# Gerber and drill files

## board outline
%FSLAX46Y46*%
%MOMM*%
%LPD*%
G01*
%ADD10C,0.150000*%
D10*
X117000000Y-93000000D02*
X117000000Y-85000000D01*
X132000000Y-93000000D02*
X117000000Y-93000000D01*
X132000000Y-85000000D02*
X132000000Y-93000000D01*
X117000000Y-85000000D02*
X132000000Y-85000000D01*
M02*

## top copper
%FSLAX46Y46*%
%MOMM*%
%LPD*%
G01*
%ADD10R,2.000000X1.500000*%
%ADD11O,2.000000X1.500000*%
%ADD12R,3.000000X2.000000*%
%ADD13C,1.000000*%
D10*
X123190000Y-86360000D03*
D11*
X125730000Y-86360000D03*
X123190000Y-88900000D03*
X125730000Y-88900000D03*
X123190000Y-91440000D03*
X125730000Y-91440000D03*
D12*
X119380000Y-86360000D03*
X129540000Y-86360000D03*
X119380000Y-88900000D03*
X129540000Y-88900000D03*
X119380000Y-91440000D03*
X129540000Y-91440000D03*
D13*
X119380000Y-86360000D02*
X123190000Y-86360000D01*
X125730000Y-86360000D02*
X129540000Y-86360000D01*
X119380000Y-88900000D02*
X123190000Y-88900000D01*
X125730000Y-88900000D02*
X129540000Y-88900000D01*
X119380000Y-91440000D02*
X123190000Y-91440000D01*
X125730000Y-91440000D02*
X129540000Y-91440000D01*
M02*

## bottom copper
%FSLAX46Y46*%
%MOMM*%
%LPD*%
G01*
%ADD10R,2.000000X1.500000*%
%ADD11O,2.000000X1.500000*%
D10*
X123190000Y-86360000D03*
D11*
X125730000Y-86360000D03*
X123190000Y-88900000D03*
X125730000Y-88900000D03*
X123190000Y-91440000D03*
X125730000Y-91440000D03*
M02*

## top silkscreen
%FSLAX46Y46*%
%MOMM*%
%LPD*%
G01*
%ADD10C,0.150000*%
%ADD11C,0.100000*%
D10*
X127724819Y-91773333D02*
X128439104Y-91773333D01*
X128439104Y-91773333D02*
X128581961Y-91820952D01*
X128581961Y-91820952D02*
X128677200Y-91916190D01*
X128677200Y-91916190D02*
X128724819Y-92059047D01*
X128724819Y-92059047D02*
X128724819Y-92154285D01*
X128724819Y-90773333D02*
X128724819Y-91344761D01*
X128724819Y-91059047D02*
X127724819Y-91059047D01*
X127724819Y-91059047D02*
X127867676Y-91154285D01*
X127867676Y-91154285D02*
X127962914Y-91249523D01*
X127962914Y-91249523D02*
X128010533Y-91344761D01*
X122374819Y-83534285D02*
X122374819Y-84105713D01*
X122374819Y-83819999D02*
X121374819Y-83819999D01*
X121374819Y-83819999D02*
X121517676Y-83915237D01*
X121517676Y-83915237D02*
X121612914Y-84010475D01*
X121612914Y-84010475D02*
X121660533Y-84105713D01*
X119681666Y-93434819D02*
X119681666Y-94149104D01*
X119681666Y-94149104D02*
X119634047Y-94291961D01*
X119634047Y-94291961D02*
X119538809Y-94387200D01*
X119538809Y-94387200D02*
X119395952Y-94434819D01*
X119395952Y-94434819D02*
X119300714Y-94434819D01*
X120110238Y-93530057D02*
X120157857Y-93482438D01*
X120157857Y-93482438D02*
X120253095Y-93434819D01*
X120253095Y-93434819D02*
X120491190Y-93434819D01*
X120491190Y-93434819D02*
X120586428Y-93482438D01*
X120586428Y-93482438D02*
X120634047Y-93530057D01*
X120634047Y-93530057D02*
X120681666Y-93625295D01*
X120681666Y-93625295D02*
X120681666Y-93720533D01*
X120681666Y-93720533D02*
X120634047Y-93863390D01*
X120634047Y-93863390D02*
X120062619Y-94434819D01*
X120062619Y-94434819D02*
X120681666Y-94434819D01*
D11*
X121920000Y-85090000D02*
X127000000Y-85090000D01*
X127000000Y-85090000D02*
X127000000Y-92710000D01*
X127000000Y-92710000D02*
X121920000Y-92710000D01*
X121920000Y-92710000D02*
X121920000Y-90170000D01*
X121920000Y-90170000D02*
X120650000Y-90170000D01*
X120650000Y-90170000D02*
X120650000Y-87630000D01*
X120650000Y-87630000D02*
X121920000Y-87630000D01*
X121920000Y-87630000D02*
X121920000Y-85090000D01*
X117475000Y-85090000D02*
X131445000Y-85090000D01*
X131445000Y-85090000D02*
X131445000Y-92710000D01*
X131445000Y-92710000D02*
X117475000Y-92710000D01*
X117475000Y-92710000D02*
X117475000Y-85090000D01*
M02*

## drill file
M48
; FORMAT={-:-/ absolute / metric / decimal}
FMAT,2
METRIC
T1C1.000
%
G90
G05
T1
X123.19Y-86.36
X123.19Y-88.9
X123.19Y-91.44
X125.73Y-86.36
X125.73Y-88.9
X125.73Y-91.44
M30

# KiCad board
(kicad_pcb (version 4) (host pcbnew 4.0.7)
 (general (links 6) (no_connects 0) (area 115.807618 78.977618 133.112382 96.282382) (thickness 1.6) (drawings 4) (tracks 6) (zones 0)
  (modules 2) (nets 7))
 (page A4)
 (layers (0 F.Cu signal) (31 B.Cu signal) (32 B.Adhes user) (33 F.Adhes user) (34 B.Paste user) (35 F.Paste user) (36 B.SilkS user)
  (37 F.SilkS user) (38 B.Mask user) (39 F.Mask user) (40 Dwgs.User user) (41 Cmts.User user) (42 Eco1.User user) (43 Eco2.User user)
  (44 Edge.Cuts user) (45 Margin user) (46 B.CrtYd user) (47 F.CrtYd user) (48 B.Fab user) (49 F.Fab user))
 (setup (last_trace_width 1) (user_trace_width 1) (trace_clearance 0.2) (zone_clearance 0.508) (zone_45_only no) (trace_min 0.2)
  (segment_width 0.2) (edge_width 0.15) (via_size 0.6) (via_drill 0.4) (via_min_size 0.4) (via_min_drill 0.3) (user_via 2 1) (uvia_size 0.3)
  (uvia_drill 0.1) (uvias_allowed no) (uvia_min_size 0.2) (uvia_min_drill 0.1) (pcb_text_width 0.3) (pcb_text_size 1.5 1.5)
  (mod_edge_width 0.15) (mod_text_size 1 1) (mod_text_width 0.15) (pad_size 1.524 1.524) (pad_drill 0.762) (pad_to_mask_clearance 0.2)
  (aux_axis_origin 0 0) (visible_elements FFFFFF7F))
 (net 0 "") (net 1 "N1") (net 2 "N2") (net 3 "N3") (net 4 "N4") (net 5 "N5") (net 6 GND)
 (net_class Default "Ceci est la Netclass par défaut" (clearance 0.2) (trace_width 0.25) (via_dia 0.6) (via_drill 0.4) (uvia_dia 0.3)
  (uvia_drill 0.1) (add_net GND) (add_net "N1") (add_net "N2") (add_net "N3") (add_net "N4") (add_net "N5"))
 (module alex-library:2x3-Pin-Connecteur (layer F.Cu) (at 123.19 86.36)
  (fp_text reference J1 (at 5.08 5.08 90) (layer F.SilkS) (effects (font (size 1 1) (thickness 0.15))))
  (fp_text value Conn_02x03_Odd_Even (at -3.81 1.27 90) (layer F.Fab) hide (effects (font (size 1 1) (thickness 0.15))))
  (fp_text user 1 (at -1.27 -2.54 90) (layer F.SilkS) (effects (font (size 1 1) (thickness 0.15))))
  (fp_line (start -1.27 -1.27) (end 3.81 -1.27) (layer F.SilkS) (width 0.1))
  (fp_line (start 3.81 -1.27) (end 3.81 6.35) (layer F.SilkS) (width 0.1))
  (fp_line (start 3.81 6.35) (end -1.27 6.35) (layer F.SilkS) (width 0.1))
  (fp_line (start -1.27 6.35) (end -1.27 3.81) (layer F.SilkS) (width 0.1))
  (fp_line (start -1.27 3.81) (end -2.54 3.81) (layer F.SilkS) (width 0.1))
  (fp_line (start -2.54 3.81) (end -2.54 1.27) (layer F.SilkS) (width 0.1))
  (fp_line (start -2.54 1.27) (end -1.27 1.27) (layer F.SilkS) (width 0.1))
  (fp_line (start -1.27 1.27) (end -1.27 -1.27) (layer F.SilkS) (width 0.1))
  (pad 1 thru_hole rect (at 0 0) (size 2 1.5) (drill 1) (layers *.Cu *.Mask) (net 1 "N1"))
  (pad 2 thru_hole oval (at 2.54 0) (size 2 1.5) (drill 1) (layers *.Cu *.Mask) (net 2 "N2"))
  (pad 3 thru_hole oval (at 0 2.54) (size 2 1.5) (drill 1) (layers *.Cu *.Mask) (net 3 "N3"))
  (pad 4 thru_hole oval (at 2.54 2.54) (size 2 1.5) (drill 1) (layers *.Cu *.Mask) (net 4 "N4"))
  (pad 5 thru_hole oval (at 0 5.08) (size 2 1.5) (drill 1) (layers *.Cu *.Mask) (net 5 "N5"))
  (pad 6 thru_hole oval (at 2.54 5.08) (size 2 1.5) (drill 1) (layers *.Cu *.Mask) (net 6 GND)))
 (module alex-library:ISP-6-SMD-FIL (layer F.Cu) (at 119.38 86.36)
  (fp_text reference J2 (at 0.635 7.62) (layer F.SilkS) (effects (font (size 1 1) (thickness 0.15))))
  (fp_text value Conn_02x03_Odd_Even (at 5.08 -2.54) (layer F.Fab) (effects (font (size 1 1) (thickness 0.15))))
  (fp_line (start -1.905 -1.27) (end 12.065 -1.27) (layer F.SilkS) (width 0.1))
  (fp_line (start 12.065 -1.27) (end 12.065 6.35) (layer F.SilkS) (width 0.1))
  (fp_line (start 12.065 6.35) (end -1.905 6.35) (layer F.SilkS) (width 0.1))
  (fp_line (start -1.905 6.35) (end -1.905 -1.27) (layer F.SilkS) (width 0.1))
  (pad 1 smd rect (at 0 0) (size 3 2) (layers F.Cu F.Paste F.Mask) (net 1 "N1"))
  (pad 2 smd rect (at 10.16 0) (size 3 2) (layers F.Cu F.Paste F.Mask) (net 2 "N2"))
  (pad 3 smd rect (at 0 2.54) (size 3 2) (layers F.Cu F.Paste F.Mask) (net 3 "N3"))
  (pad 4 smd rect (at 10.16 2.54) (size 3 2) (layers F.Cu F.Paste F.Mask) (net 4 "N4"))
  (pad 5 smd rect (at 0 5.08) (size 3 2) (layers F.Cu F.Paste F.Mask) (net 5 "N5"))
  (pad 6 smd rect (at 10.16 5.08) (size 3 2) (layers F.Cu F.Paste F.Mask) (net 6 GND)))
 (gr_line (start 117 93) (end 117 85) (angle 90) (layer Edge.Cuts) (width 0.15))
 (gr_line (start 132 93) (end 117 93) (angle 90) (layer Edge.Cuts) (width 0.15))
 (gr_line (start 132 85) (end 132 93) (angle 90) (layer Edge.Cuts) (width 0.15))
 (gr_line (start 117 85) (end 132 85) (angle 90) (layer Edge.Cuts) (width 0.15))
 (segment (start 119.38 86.36) (end 123.19 86.36) (width 1) (layer F.Cu) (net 1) (status C00000))
 (segment (start 125.73 86.36) (end 129.54 86.36) (width 1) (layer F.Cu) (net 2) (status C00000))
 (segment (start 119.38 88.9) (end 123.19 88.9) (width 1) (layer F.Cu) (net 3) (status C00000))
 (segment (start 125.73 88.9) (end 129.54 88.9) (width 1) (layer F.Cu) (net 4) (status C00000))
 (segment (start 119.38 91.44) (end 123.19 91.44) (width 1) (layer F.Cu) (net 5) (status C00000))
 (segment (start 125.73 91.44) (end 129.54 91.44) (width 1) (layer F.Cu) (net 6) (status C00000)))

